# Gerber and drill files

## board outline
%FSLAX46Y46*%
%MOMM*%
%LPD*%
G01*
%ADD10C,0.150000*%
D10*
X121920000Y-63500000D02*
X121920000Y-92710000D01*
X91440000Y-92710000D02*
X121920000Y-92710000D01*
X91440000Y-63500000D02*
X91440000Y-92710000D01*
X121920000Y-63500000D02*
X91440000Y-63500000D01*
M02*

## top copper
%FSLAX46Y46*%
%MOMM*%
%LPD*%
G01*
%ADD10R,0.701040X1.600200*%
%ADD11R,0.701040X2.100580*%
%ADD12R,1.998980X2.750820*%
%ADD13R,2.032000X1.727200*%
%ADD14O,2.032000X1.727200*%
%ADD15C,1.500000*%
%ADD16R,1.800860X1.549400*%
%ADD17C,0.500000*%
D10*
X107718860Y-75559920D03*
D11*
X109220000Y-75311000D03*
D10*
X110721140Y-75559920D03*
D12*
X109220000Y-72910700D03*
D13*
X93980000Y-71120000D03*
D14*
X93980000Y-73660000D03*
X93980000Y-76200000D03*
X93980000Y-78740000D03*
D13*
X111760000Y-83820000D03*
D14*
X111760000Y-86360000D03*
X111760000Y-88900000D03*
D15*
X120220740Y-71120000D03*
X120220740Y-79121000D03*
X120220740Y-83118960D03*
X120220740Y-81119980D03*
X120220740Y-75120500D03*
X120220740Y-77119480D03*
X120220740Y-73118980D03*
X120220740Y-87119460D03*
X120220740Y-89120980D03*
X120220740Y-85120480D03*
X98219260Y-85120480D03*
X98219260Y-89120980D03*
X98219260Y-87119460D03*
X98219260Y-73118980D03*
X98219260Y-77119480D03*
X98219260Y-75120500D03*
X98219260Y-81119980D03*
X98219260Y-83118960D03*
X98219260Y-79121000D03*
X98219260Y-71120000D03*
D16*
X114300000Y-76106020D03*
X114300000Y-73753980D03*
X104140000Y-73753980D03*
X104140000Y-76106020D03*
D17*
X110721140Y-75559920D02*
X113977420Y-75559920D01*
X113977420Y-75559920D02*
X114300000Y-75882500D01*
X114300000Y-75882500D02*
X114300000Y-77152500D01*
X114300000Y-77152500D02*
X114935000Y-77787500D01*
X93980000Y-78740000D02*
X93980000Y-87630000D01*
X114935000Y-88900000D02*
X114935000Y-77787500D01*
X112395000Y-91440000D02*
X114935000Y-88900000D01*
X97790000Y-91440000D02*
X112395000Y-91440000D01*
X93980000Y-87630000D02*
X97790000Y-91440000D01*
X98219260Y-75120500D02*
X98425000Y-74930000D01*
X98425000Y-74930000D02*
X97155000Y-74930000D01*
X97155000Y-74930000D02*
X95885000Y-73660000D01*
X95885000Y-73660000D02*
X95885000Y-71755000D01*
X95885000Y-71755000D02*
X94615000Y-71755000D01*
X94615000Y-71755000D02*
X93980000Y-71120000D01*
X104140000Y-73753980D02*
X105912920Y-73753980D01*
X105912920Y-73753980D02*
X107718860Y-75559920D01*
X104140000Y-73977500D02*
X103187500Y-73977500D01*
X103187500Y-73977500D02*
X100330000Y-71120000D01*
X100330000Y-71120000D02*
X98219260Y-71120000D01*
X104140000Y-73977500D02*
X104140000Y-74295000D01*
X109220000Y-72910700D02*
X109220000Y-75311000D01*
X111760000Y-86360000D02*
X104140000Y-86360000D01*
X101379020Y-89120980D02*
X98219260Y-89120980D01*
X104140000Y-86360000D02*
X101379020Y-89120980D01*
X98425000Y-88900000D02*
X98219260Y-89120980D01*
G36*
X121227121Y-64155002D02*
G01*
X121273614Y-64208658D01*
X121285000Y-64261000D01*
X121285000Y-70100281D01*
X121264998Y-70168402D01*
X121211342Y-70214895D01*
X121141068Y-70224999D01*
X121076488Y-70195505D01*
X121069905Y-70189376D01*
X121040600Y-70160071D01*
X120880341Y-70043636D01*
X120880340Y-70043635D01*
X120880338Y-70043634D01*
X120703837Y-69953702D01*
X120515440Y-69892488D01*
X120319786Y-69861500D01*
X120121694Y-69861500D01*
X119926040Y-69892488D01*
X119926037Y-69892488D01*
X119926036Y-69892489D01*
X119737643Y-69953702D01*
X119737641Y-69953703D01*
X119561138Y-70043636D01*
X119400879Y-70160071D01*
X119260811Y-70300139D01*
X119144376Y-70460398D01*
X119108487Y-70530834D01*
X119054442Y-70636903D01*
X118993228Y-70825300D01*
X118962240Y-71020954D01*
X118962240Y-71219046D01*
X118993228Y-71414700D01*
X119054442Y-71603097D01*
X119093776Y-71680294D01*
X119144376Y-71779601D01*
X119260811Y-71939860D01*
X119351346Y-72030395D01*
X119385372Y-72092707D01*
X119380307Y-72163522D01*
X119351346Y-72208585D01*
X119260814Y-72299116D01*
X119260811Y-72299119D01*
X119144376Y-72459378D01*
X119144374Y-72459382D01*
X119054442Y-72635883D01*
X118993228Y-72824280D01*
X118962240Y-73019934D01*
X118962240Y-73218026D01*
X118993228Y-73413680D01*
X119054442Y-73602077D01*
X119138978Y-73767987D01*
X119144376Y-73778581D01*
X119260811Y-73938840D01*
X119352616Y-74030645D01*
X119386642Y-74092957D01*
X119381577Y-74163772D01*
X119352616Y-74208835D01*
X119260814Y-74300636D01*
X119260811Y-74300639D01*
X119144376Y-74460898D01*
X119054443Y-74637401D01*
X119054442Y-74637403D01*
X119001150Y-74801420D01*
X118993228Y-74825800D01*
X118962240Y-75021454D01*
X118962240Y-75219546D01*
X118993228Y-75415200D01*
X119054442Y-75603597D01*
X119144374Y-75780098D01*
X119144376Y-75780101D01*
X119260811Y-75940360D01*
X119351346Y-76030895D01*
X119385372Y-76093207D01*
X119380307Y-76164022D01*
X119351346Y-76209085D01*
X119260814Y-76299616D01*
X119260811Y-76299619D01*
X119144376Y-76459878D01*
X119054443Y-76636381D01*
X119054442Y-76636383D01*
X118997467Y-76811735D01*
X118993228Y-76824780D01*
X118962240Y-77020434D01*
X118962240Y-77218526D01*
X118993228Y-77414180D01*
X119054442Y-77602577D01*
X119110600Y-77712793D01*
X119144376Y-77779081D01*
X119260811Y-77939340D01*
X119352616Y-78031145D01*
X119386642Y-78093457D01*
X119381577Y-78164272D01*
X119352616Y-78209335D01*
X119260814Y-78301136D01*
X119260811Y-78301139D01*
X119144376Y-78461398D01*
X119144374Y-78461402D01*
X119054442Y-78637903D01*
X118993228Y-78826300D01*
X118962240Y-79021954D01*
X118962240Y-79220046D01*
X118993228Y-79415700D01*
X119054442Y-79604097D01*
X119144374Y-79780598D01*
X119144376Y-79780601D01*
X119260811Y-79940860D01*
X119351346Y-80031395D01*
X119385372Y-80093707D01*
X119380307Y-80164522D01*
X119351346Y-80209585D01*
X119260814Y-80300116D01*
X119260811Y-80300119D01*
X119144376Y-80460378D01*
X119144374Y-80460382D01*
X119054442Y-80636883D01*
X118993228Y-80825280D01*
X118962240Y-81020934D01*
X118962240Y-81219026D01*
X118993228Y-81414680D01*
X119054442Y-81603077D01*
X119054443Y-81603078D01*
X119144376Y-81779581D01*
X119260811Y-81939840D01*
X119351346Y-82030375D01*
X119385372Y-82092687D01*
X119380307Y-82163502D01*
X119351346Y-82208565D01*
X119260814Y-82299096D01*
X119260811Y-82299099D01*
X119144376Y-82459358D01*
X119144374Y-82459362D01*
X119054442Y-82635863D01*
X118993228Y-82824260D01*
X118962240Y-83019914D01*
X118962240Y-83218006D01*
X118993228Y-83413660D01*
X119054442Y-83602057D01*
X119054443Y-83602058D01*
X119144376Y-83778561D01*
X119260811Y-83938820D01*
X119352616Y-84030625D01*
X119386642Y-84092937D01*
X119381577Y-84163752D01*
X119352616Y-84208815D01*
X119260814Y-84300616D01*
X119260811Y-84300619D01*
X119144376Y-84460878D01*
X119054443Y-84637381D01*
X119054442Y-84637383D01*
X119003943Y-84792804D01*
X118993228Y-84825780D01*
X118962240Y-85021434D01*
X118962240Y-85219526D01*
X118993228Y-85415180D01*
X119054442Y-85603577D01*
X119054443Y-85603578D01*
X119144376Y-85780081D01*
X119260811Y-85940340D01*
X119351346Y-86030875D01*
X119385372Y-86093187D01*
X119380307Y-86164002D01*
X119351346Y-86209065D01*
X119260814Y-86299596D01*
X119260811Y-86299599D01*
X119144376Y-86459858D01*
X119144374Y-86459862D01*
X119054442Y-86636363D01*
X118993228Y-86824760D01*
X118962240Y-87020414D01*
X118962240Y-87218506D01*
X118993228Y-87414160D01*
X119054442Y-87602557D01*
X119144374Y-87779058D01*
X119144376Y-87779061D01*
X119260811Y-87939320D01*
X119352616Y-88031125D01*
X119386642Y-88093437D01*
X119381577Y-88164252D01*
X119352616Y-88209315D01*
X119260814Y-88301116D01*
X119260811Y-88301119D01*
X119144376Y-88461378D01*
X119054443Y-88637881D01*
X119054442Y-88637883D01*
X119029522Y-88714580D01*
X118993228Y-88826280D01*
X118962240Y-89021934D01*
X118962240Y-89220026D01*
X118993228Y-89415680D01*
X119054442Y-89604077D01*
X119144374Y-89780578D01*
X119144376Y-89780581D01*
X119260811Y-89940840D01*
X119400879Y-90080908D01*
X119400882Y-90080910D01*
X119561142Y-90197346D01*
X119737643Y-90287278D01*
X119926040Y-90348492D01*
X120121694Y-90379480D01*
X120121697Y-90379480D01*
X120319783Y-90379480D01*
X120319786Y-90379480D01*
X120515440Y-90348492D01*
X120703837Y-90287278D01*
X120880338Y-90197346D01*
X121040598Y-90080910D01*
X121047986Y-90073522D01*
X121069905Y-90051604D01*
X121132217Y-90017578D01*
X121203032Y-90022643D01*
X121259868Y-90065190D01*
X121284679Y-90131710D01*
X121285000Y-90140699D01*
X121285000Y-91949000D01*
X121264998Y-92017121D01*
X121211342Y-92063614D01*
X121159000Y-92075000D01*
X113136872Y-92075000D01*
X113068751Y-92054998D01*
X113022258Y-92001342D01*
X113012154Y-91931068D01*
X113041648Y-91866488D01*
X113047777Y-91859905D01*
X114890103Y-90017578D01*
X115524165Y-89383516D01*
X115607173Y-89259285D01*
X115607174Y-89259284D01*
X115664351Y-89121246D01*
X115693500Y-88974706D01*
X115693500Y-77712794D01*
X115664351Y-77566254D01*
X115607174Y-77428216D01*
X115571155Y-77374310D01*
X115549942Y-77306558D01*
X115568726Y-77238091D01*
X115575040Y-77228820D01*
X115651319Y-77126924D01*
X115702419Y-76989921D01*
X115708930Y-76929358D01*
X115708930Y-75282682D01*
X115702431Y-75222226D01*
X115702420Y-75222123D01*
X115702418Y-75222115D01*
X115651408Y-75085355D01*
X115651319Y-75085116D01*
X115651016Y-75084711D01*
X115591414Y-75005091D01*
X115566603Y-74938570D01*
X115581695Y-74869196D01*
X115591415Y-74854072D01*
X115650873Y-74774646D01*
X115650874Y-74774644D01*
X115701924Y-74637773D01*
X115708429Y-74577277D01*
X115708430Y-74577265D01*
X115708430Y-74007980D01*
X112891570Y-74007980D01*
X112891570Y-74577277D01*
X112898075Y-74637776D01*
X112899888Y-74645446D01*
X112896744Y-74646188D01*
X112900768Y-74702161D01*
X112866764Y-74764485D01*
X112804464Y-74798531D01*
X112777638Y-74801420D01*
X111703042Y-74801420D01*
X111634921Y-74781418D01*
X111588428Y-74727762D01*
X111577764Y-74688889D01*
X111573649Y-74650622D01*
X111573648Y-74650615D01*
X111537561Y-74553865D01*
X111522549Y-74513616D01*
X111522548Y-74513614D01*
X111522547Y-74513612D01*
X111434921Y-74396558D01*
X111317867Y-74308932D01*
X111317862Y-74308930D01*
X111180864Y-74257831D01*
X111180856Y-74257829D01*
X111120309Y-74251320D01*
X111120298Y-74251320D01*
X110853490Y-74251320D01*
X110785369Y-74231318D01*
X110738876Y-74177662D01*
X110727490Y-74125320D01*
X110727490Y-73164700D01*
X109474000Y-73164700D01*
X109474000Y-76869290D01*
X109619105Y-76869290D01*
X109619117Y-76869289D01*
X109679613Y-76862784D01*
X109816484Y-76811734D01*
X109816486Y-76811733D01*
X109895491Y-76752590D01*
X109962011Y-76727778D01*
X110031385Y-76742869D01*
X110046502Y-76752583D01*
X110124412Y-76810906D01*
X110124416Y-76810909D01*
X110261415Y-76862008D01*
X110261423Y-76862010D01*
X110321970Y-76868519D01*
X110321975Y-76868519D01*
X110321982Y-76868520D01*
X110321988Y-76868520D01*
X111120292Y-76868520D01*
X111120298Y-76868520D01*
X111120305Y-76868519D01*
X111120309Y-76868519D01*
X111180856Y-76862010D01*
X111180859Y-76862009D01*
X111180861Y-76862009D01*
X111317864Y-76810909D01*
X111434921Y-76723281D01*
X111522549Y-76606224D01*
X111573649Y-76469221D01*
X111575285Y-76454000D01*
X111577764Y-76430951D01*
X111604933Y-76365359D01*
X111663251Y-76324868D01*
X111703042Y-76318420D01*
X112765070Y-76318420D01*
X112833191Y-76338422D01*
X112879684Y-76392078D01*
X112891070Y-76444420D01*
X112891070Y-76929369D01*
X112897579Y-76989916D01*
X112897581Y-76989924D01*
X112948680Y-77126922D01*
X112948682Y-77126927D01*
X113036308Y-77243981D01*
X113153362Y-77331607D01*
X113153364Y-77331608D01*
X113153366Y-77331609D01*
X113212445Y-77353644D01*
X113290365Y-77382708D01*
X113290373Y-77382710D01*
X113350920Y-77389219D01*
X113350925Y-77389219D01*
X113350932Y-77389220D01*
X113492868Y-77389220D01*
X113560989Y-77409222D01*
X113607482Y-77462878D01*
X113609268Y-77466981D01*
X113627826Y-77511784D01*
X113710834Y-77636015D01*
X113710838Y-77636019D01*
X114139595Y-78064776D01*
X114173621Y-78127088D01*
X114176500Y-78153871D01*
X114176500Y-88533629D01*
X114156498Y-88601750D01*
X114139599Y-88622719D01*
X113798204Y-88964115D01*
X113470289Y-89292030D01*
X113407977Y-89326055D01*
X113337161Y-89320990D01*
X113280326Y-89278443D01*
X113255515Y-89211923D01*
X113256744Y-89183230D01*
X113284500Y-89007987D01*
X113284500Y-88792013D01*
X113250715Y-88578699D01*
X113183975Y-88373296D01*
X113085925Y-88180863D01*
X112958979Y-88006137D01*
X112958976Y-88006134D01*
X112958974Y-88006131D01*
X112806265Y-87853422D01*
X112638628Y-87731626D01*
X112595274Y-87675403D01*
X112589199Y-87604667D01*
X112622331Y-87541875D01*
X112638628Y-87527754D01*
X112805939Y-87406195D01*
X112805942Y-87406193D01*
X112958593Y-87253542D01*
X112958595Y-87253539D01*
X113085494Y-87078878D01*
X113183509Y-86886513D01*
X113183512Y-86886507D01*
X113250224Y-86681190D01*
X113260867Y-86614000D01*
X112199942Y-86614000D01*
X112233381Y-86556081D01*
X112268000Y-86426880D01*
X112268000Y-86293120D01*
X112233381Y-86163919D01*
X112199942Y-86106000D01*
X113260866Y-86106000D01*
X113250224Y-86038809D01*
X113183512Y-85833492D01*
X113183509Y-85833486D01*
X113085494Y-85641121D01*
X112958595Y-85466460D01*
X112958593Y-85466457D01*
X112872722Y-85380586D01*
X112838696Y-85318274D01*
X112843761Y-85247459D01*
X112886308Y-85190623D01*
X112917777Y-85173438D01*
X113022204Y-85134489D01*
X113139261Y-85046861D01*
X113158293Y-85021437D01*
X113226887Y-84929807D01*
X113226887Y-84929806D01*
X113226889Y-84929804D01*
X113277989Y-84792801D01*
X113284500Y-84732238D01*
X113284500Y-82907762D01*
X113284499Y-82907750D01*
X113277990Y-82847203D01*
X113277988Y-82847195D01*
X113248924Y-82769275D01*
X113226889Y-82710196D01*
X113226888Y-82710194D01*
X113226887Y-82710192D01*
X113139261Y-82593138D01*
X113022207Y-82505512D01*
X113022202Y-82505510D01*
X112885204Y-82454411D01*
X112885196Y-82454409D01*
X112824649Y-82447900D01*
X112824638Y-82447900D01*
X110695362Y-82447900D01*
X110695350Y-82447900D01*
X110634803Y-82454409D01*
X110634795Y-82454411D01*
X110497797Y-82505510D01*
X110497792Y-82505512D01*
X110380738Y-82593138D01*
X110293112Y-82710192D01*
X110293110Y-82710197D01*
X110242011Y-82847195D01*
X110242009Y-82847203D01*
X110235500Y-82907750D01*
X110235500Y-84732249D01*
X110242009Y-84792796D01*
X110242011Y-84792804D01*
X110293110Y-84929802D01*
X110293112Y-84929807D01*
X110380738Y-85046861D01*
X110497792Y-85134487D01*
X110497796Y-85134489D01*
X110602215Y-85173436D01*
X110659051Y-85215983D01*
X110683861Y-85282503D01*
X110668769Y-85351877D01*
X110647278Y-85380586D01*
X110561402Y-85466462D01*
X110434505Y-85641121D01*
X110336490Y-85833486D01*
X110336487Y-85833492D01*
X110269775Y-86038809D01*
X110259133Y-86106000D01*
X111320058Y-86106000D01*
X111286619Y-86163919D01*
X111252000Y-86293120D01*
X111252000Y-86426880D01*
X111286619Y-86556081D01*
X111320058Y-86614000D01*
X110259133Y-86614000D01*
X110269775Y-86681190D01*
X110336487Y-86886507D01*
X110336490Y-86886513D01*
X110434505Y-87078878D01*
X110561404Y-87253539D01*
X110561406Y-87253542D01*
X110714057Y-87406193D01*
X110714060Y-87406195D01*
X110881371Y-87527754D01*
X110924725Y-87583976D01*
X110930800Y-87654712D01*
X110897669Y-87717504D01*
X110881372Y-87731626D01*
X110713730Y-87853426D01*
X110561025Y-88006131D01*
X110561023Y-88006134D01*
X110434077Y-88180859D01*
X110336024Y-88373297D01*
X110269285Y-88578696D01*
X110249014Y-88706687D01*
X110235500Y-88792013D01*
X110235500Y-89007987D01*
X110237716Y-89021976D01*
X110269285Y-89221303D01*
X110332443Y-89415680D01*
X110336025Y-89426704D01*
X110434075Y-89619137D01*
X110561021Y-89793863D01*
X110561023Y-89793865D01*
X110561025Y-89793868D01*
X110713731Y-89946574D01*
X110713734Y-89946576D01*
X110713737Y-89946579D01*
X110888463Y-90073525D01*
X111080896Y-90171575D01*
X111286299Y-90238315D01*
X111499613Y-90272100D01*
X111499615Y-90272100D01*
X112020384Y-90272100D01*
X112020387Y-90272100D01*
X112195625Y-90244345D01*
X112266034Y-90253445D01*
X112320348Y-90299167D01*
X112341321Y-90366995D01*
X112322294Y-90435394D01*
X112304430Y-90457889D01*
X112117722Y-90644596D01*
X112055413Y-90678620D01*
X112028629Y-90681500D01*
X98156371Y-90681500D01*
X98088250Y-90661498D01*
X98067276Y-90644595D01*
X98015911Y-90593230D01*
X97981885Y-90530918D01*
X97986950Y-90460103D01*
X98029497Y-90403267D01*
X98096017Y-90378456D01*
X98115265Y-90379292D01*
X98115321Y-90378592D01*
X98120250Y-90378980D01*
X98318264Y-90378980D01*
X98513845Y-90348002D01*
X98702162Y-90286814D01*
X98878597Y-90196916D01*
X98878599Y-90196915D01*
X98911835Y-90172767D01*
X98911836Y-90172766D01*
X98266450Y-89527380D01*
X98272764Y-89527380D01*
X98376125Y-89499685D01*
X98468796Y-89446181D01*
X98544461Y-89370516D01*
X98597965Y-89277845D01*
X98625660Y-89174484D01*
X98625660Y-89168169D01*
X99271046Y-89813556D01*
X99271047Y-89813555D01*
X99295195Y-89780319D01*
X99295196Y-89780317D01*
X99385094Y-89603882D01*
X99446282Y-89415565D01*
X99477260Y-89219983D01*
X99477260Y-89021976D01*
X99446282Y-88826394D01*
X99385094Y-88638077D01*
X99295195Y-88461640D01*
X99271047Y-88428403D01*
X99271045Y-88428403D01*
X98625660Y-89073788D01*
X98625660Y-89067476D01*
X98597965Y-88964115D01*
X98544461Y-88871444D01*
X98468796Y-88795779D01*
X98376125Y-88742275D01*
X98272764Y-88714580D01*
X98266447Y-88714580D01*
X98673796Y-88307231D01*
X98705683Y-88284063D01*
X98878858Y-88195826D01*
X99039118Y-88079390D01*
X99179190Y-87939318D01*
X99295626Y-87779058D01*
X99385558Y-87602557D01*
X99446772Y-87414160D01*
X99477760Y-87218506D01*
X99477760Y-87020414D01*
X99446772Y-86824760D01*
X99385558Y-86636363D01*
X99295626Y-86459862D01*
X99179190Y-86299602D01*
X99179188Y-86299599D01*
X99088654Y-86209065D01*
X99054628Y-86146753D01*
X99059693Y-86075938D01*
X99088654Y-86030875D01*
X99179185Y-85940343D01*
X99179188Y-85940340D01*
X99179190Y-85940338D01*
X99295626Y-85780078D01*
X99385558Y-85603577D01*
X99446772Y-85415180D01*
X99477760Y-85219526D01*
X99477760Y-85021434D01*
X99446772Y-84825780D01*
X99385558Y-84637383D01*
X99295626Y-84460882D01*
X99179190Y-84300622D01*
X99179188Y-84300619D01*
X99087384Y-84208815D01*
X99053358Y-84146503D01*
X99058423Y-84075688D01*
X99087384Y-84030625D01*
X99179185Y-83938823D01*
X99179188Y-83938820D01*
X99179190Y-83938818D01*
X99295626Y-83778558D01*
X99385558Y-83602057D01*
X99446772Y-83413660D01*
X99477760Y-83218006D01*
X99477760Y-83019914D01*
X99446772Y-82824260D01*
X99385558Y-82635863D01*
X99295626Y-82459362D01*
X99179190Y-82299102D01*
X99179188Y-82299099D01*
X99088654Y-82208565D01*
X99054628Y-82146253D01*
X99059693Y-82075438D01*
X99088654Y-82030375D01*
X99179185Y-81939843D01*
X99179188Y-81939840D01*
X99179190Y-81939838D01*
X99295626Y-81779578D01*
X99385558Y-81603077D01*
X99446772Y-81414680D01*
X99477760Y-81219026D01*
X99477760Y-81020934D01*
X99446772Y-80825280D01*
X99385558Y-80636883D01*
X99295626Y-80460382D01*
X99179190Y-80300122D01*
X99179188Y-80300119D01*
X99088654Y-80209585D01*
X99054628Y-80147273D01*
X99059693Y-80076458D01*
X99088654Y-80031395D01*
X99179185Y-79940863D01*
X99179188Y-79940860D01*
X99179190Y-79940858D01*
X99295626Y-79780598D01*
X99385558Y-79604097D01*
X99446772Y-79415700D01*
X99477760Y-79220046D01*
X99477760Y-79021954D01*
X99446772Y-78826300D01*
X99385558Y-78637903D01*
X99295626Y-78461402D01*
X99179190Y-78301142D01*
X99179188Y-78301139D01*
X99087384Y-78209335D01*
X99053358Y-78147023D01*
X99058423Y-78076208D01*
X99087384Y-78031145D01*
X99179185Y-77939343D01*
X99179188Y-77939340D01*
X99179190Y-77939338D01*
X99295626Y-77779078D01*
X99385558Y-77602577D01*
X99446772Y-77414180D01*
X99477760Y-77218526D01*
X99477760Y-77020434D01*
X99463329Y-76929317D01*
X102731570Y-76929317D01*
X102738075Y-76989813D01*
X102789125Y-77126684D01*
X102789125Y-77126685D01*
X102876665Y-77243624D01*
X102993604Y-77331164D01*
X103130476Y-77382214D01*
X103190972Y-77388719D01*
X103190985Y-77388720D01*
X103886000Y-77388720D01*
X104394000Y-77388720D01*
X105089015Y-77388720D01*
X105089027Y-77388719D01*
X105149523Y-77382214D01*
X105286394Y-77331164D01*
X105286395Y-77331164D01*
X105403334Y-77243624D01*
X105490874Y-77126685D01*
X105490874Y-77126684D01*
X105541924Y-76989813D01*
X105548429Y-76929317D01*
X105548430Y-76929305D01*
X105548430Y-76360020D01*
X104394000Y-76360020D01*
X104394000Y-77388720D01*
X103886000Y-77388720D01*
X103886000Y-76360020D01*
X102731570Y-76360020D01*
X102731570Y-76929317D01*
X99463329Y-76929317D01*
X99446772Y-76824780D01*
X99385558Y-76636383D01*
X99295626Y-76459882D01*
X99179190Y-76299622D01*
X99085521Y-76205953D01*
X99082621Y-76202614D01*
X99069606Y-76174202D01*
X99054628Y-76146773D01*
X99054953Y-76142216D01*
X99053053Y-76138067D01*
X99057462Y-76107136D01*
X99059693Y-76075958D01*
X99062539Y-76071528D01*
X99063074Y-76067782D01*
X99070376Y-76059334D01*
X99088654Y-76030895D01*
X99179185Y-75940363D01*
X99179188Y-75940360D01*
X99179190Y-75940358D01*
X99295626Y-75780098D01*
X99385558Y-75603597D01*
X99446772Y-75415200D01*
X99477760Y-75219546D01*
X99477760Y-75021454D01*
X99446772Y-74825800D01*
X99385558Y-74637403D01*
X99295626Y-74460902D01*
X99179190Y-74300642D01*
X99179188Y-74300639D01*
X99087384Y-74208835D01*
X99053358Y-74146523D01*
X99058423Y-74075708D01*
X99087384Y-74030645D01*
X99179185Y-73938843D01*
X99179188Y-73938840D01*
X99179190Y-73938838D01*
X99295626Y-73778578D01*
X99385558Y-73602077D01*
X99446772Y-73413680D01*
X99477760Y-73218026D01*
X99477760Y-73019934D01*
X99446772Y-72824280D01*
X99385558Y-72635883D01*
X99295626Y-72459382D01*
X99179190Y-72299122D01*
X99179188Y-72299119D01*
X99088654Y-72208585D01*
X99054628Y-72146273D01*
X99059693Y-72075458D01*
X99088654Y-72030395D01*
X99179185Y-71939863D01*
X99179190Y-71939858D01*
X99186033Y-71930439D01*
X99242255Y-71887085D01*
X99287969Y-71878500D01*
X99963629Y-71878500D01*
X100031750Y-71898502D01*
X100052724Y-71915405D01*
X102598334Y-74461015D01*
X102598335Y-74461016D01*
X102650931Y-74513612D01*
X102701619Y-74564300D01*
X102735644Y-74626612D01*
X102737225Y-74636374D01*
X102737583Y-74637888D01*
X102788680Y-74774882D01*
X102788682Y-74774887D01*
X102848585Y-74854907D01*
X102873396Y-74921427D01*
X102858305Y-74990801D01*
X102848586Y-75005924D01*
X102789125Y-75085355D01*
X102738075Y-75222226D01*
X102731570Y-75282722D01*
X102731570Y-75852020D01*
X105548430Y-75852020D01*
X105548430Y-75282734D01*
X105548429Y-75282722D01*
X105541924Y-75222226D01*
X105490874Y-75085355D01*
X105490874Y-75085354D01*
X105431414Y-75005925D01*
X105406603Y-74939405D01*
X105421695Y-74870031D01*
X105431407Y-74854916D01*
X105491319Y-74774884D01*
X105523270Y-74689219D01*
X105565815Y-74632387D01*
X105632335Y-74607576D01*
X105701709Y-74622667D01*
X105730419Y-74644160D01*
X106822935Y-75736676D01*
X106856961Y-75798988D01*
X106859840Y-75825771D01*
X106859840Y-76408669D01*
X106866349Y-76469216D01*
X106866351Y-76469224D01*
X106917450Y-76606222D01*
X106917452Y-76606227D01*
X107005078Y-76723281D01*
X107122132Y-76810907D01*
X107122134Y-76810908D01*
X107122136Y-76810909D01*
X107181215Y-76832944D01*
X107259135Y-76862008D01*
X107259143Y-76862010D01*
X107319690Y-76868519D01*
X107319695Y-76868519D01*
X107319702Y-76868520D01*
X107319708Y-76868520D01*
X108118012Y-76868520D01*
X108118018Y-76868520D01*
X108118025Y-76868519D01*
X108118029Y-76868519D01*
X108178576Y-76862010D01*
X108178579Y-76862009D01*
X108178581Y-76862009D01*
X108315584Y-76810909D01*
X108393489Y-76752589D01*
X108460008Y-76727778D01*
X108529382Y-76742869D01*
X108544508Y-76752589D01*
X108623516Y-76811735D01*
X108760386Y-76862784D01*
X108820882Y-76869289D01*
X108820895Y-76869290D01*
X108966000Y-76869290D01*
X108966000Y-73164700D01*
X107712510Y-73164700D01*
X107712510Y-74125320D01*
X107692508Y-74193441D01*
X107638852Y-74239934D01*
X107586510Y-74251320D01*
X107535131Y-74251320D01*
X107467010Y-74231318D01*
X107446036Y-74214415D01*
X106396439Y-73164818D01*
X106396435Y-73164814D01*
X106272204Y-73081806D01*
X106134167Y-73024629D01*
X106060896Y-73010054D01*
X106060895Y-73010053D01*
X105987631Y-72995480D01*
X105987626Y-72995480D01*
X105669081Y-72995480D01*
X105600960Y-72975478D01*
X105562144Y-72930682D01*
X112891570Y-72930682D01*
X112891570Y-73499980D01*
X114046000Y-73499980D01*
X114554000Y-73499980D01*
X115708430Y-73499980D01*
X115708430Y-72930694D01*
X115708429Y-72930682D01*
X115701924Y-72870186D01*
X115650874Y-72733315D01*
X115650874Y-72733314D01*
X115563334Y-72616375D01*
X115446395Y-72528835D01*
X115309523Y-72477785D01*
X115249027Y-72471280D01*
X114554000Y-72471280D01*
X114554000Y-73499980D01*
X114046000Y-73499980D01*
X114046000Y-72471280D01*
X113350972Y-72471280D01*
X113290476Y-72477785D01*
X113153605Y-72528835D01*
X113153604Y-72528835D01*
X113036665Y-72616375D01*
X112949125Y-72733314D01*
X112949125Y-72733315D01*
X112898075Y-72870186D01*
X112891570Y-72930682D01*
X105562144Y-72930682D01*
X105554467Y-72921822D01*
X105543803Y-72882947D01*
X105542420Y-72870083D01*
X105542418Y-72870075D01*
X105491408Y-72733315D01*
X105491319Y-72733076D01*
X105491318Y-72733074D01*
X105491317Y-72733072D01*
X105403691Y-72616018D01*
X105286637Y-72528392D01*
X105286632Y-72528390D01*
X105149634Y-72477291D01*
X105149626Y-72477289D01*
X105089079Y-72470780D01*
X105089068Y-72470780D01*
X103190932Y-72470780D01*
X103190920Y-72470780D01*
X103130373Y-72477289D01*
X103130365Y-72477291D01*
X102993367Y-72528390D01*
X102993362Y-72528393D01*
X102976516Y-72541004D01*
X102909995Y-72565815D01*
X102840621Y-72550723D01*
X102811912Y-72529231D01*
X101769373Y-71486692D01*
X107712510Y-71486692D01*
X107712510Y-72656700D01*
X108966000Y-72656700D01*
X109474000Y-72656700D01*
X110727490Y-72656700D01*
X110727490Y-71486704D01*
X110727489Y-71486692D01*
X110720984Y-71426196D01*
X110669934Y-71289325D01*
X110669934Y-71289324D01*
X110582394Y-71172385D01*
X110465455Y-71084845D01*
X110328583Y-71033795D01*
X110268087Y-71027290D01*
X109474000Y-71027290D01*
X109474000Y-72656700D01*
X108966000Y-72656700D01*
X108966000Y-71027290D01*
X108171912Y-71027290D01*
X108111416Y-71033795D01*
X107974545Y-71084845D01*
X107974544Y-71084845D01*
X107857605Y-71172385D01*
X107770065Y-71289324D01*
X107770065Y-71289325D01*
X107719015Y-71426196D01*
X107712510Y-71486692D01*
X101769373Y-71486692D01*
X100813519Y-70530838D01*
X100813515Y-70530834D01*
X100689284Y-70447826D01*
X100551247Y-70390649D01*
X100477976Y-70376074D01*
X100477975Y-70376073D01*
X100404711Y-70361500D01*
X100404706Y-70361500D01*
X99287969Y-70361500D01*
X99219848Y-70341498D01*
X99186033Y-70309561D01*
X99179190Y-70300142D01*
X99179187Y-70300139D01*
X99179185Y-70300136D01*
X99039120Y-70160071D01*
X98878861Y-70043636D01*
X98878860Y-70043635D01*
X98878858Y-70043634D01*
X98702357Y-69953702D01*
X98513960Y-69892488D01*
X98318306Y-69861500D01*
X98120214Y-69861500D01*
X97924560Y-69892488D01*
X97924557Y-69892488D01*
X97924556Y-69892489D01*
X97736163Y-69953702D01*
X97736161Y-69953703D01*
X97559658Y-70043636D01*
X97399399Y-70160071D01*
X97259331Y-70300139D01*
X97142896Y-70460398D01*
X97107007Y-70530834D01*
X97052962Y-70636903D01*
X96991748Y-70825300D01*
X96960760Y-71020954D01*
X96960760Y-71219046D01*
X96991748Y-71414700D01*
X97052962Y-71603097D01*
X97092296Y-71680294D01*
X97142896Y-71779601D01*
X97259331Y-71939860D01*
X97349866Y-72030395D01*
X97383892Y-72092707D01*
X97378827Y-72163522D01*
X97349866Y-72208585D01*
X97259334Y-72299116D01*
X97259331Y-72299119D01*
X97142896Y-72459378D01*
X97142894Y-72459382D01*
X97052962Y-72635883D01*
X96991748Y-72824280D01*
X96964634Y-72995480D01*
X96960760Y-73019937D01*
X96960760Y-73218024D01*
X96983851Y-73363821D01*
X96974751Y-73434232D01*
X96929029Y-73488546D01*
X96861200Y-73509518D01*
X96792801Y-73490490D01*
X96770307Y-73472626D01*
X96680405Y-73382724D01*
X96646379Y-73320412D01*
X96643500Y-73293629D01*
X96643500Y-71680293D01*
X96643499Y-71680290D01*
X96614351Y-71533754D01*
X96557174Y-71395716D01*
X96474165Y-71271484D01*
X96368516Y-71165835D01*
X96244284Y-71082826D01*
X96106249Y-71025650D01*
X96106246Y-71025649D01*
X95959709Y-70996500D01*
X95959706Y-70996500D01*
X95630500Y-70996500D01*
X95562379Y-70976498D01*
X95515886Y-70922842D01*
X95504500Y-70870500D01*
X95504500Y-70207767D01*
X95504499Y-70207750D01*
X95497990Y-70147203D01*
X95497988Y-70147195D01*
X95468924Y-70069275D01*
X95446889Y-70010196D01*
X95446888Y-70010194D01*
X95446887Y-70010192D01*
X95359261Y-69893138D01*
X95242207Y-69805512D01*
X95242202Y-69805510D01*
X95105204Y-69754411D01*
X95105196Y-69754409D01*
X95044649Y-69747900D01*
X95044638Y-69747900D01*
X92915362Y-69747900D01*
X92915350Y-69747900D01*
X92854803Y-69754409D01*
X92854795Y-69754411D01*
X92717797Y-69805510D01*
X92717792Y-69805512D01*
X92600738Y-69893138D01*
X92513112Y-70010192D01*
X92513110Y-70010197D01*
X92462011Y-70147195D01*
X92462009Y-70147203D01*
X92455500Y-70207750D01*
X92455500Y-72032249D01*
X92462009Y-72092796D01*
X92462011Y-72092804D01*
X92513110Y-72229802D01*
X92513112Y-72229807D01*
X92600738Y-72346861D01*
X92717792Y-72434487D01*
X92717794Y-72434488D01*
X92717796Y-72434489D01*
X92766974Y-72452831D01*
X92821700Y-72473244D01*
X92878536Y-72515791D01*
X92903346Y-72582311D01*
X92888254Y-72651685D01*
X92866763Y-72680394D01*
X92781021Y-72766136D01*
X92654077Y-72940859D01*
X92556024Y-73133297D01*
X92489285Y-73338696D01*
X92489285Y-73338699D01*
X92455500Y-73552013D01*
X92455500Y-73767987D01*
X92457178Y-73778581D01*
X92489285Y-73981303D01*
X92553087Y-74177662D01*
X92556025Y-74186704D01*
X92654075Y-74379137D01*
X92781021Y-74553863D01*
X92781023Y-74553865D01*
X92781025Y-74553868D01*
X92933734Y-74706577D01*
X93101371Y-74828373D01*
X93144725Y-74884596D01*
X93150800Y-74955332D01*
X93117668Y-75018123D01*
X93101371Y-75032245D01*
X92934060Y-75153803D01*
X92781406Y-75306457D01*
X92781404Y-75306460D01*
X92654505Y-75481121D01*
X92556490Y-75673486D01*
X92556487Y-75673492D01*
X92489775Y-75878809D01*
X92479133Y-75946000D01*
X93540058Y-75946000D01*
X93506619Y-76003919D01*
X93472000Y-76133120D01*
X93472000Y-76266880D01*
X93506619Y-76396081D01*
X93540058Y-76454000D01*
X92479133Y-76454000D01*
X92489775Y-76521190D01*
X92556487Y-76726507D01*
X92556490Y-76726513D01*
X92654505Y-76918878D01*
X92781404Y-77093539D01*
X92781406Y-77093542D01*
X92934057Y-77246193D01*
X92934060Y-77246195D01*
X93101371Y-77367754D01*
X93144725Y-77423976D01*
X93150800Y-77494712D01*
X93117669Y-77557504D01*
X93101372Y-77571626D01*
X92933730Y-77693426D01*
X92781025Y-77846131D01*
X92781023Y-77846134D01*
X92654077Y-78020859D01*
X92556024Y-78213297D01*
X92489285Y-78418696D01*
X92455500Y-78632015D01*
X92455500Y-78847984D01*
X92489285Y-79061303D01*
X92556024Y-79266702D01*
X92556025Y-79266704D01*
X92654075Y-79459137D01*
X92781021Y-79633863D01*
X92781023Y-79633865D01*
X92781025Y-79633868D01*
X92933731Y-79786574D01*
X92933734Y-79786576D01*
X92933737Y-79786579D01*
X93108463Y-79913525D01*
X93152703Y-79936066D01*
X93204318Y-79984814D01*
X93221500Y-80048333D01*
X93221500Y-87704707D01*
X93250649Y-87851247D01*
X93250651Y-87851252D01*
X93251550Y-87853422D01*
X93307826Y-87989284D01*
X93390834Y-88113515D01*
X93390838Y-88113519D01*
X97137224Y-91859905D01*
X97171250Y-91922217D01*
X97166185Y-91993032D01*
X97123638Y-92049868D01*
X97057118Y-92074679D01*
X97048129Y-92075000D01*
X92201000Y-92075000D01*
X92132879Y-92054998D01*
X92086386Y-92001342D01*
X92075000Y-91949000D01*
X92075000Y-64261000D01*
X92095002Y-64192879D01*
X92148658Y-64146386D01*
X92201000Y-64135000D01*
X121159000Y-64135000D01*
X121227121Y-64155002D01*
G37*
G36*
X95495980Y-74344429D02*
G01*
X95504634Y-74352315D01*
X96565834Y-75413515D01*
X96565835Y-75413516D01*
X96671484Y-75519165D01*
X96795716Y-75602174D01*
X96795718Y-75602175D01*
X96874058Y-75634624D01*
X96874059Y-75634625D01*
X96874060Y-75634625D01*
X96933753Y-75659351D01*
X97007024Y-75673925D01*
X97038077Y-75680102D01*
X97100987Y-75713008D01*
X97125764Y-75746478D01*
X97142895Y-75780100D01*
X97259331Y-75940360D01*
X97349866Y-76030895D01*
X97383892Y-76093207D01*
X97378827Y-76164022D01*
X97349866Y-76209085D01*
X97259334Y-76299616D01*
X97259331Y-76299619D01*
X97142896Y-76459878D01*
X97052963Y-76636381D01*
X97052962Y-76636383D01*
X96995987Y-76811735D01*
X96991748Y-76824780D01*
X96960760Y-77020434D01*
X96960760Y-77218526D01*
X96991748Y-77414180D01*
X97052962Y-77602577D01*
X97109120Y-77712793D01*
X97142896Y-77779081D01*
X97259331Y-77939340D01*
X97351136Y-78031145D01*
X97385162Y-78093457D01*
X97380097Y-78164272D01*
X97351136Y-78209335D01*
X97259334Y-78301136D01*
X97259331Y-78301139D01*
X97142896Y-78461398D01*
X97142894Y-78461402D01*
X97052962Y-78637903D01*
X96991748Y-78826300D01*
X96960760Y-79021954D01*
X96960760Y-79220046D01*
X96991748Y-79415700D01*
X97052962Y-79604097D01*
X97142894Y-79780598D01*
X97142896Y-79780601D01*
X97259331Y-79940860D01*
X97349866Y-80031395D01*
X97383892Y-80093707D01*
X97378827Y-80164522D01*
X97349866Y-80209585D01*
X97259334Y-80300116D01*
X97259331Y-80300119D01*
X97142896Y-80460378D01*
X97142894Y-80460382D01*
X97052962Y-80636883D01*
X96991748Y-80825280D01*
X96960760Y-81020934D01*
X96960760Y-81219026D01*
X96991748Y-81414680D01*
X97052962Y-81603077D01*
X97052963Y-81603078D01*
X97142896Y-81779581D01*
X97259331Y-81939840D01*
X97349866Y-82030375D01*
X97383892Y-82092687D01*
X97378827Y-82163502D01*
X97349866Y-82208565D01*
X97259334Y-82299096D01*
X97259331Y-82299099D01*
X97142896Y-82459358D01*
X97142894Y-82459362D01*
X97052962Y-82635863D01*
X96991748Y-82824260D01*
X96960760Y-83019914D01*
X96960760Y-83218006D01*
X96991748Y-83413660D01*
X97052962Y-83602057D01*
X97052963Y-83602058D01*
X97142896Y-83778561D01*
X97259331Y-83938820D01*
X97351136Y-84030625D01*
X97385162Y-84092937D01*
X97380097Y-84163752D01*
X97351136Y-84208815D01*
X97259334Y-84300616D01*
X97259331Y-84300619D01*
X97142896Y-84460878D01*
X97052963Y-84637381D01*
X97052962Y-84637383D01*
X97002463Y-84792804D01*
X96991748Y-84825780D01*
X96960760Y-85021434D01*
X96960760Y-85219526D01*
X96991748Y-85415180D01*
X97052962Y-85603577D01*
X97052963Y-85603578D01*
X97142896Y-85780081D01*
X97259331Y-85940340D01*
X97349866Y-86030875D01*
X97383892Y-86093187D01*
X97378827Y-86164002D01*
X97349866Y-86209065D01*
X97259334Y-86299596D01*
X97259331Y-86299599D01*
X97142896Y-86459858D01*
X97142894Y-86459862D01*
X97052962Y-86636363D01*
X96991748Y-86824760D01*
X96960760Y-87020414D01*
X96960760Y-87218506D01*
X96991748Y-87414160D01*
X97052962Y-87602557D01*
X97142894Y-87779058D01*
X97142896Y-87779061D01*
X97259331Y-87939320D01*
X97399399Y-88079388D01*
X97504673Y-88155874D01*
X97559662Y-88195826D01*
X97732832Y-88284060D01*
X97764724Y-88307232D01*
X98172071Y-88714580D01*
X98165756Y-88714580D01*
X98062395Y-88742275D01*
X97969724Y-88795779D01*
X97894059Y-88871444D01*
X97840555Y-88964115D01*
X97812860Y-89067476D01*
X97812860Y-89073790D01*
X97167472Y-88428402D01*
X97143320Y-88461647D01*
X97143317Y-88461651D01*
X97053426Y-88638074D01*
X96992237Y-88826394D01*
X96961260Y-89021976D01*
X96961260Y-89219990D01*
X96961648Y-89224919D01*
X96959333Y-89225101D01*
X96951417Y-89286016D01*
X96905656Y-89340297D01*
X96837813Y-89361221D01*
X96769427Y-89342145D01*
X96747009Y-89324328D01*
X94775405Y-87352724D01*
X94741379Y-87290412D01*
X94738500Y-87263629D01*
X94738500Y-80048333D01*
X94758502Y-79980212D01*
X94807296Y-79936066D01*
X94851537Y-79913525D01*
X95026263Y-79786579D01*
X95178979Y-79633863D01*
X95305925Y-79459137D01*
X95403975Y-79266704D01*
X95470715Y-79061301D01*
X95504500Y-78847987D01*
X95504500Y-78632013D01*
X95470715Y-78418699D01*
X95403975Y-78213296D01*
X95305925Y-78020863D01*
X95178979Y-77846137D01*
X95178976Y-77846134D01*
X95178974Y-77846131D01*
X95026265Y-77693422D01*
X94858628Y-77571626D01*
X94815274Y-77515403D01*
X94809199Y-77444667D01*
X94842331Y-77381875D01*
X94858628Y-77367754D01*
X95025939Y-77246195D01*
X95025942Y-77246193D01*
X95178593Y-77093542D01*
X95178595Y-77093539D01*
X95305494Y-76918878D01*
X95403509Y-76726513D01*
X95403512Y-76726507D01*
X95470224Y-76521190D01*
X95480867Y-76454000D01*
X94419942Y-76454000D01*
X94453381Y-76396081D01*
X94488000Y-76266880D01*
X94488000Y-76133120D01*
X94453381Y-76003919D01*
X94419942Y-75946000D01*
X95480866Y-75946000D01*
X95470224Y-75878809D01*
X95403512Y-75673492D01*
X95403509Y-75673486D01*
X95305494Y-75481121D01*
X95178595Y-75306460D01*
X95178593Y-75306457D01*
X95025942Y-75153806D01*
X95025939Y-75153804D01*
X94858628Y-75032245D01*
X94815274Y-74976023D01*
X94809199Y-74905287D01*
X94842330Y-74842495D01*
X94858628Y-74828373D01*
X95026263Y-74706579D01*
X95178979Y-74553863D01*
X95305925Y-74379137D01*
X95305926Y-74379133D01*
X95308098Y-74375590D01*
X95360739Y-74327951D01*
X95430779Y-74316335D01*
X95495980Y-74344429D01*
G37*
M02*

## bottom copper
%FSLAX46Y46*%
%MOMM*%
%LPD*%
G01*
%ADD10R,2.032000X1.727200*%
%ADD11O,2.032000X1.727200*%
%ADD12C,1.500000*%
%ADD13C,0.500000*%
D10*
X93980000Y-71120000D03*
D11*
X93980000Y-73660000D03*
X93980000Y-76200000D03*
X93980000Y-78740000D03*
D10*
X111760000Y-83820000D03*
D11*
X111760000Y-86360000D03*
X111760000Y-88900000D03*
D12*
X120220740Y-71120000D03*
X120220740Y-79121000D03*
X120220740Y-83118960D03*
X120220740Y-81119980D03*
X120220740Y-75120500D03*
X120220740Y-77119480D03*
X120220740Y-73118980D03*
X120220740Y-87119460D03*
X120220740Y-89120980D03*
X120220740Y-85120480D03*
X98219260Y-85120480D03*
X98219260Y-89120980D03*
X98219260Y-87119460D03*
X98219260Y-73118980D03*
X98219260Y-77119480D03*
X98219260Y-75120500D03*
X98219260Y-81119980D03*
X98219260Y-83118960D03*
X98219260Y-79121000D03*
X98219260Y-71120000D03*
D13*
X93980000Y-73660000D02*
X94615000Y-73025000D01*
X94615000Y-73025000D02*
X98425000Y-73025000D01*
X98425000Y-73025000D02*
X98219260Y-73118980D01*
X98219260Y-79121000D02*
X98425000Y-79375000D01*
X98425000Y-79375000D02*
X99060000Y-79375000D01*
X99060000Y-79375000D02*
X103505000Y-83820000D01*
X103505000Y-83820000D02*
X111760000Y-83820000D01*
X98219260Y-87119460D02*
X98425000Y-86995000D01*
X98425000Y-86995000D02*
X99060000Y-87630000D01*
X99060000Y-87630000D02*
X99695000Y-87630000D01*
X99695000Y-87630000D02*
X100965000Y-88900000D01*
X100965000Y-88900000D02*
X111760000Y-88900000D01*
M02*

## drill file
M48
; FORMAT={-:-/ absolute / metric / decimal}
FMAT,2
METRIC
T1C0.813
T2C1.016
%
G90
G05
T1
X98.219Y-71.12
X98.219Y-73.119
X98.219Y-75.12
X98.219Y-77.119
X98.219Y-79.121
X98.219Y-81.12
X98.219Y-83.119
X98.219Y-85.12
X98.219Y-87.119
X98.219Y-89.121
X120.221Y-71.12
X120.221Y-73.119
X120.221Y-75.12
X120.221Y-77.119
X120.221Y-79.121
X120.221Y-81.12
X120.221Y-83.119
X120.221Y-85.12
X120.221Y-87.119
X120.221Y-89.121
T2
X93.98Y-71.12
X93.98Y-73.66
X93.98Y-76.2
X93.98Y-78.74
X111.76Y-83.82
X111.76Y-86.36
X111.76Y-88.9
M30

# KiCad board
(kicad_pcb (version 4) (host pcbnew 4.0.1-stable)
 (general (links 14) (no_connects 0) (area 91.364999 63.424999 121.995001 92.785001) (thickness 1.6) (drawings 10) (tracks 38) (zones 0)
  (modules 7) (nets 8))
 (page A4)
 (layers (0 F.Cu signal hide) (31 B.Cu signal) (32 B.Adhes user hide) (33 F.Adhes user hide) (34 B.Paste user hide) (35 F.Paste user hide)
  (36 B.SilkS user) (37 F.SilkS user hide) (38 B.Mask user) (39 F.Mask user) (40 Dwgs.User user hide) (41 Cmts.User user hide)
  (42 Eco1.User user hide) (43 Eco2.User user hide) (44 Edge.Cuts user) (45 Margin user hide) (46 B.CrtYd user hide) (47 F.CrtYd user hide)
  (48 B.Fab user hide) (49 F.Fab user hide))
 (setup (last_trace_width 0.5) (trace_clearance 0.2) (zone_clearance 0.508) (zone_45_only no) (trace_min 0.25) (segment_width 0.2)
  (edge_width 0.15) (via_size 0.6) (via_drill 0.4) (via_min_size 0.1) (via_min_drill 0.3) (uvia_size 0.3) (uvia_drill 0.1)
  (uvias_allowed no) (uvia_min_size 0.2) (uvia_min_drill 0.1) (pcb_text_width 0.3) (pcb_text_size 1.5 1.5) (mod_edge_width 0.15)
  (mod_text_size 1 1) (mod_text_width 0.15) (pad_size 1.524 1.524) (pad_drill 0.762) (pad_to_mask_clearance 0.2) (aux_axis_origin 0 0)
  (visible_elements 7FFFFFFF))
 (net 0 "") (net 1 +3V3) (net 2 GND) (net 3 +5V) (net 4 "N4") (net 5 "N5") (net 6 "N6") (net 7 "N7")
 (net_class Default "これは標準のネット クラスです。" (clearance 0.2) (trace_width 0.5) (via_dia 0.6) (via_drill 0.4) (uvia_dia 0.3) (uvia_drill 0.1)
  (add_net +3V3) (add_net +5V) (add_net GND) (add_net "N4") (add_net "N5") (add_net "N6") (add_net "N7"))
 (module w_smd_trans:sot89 (layer F.Cu) (at 109.22 73.66)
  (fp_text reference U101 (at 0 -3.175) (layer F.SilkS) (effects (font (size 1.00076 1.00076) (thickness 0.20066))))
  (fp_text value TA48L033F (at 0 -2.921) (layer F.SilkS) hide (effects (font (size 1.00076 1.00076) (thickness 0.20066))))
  (pad 1 smd rect (at -1.50114 1.89992) (size 0.70104 1.6002) (layers F.Cu F.Paste F.Mask) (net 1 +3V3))
  (pad 2 smd rect (at 0 1.651) (size 0.70104 2.10058) (layers F.Cu F.Paste F.Mask) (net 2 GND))
  (pad 3 smd rect (at 1.50114 1.89992) (size 0.70104 1.6002) (layers F.Cu F.Paste F.Mask) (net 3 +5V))
  (pad 2 smd rect (at 0 -0.7493) (size 1.99898 2.75082) (layers F.Cu F.Paste F.Mask) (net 2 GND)))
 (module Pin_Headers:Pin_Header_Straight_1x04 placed (layer B.Cu) (at 93.98 71.12 180)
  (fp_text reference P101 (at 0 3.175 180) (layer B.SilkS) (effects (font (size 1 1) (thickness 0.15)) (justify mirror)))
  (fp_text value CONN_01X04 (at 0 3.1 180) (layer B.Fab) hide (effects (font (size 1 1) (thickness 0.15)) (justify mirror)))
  (pad 1 thru_hole rect (at 0 0 180) (size 2.032 1.7272) (drill 1.016) (layers *.Cu *.Mask B.SilkS) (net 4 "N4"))
  (pad 2 thru_hole oval (at 0 -2.54 180) (size 2.032 1.7272) (drill 1.016) (layers *.Cu *.Mask B.SilkS) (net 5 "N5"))
  (pad 3 thru_hole oval (at 0 -5.08 180) (size 2.032 1.7272) (drill 1.016) (layers *.Cu *.Mask B.SilkS) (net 2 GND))
  (pad 4 thru_hole oval (at 0 -7.62 180) (size 2.032 1.7272) (drill 1.016) (layers *.Cu *.Mask B.SilkS) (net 3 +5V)))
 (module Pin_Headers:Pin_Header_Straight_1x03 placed (layer B.Cu) (at 111.76 83.82 180)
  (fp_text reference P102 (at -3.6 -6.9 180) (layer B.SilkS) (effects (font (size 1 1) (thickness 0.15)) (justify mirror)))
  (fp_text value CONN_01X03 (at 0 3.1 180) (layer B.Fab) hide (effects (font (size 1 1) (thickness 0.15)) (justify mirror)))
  (pad 1 thru_hole rect (at 0 0 180) (size 2.032 1.7272) (drill 1.016) (layers *.Cu *.Mask B.SilkS) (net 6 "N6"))
  (pad 2 thru_hole oval (at 0 -2.54 180) (size 2.032 1.7272) (drill 1.016) (layers *.Cu *.Mask B.SilkS) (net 2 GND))
  (pad 3 thru_hole oval (at 0 -5.08 180) (size 2.032 1.7272) (drill 1.016) (layers *.Cu *.Mask B.SilkS) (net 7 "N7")))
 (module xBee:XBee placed (layer F.Cu) (at 109.22 71.12)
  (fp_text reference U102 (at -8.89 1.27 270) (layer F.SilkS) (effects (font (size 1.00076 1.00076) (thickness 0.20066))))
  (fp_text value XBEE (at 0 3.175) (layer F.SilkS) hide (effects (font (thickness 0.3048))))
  (pad 20 thru_hole circle (at 11.00074 0) (size 1.5 1.5) (drill 0.8128) (layers *.Cu))
  (pad 16 thru_hole circle (at 11.00074 8.001) (size 1.5 1.5) (drill 0.8128) (layers *.Cu))
  (pad 14 thru_hole circle (at 11.00074 11.99896) (size 1.5 1.5) (drill 0.8128) (layers *.Cu))
  (pad 15 thru_hole circle (at 11.00074 9.99998) (size 1.5 1.5) (drill 0.8128) (layers *.Cu))
  (pad 18 thru_hole circle (at 11.00074 4.0005) (size 1.5 1.5) (drill 0.8128) (layers *.Cu))
  (pad 17 thru_hole circle (at 11.00074 5.99948) (size 1.5 1.5) (drill 0.8128) (layers *.Cu))
  (pad 19 thru_hole circle (at 11.00074 1.99898) (size 1.5 1.5) (drill 0.8128) (layers *.Cu))
  (pad 12 thru_hole circle (at 11.00074 15.99946) (size 1.5 1.5) (drill 0.8128) (layers *.Cu))
  (pad 11 thru_hole circle (at 11.00074 18.00098) (size 1.5 1.5) (drill 0.8128) (layers *.Cu))
  (pad 13 thru_hole circle (at 11.00074 14.00048) (size 1.5 1.5) (drill 0.8128) (layers *.Cu))
  (pad 8 thru_hole circle (at -11.00074 14.00048) (size 1.5 1.5) (drill 0.8128) (layers *.Cu))
  (pad 10 thru_hole circle (at -11.00074 18.00098) (size 1.5 1.5) (drill 0.8128) (layers *.Cu) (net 2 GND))
  (pad 9 thru_hole circle (at -11.00074 15.99946) (size 1.5 1.5) (drill 0.8128) (layers *.Cu) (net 7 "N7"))
  (pad 2 thru_hole circle (at -11.00074 1.99898) (size 1.5 1.5) (drill 0.8128) (layers *.Cu) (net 5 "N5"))
  (pad 4 thru_hole circle (at -11.00074 5.99948) (size 1.5 1.5) (drill 0.8128) (layers *.Cu))
  (pad 3 thru_hole circle (at -11.00074 4.0005) (size 1.5 1.5) (drill 0.8128) (layers *.Cu) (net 4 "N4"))
  (pad 6 thru_hole circle (at -11.00074 9.99998) (size 1.5 1.5) (drill 0.8128) (layers *.Cu))
  (pad 7 thru_hole circle (at -11.00074 11.99896) (size 1.5 1.5) (drill 0.8128) (layers *.Cu))
  (pad 5 thru_hole circle (at -11.00074 8.001) (size 1.5 1.5) (drill 0.8128) (layers *.Cu) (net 6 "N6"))
  (pad 1 thru_hole circle (at -11.00074 0) (size 1.5 1.5) (drill 0.8128) (layers *.Cu) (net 1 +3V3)))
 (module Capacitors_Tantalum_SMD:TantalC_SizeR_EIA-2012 (layer F.Cu) (at 114.3 74.93 270)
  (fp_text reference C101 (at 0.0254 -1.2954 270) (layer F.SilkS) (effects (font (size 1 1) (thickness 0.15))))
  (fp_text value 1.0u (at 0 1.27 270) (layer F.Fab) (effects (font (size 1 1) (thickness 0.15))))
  (pad 1 smd rect (at 1.17602 0 270) (size 1.5494 1.80086) (layers F.Cu F.Paste F.Mask) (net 3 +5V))
  (pad 2 smd rect (at -1.17602 0 270) (size 1.5494 1.80086) (layers F.Cu F.Paste F.Mask) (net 2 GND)))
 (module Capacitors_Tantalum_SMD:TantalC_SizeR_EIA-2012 (layer F.Cu) (at 104.14 74.93 90)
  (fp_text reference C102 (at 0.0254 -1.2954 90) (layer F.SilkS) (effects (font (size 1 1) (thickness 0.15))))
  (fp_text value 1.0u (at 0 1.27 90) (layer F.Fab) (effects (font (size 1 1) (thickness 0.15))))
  (pad 1 smd rect (at 1.17602 0 90) (size 1.5494 1.80086) (layers F.Cu F.Paste F.Mask) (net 1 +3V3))
  (pad 2 smd rect (at -1.17602 0 90) (size 1.5494 1.80086) (layers F.Cu F.Paste F.Mask) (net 2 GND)))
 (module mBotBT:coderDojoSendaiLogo (layer B.Cu) (at 107.442 73.152 180)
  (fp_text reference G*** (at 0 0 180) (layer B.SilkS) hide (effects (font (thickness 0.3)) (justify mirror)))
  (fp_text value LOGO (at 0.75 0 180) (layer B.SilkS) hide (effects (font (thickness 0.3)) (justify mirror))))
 (gr_line (start 121.92 63.5) (end 121.92 92.71) (angle 90) (layer Edge.Cuts) (width 0.15))
 (gr_line (start 91.44 92.71) (end 121.92 92.71) (angle 90) (layer Edge.Cuts) (width 0.15))
 (gr_line (start 91.44 63.5) (end 91.44 92.71) (angle 90) (layer Edge.Cuts) (width 0.15))
 (gr_line (start 121.92 63.5) (end 91.44 63.5) (angle 90) (layer Edge.Cuts) (width 0.15))
 (segment (start 110.72114 75.55992) (end 113.97742 75.55992) (width 0.5) (layer F.Cu) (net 3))
 (segment (start 113.97742 75.55992) (end 114.3 75.8825) (width 0.5) (layer F.Cu) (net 3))
 (segment (start 114.3 75.8825) (end 114.3 77.1525) (width 0.5) (layer F.Cu) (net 3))
 (segment (start 114.3 77.1525) (end 114.935 77.7875) (width 0.5) (layer F.Cu) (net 3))
 (segment (start 93.98 78.74) (end 93.98 87.63) (width 0.5) (layer F.Cu) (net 3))
 (segment (start 114.935 88.9) (end 114.935 77.7875) (width 0.5) (layer F.Cu) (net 3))
 (segment (start 112.395 91.44) (end 114.935 88.9) (width 0.5) (layer F.Cu) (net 3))
 (segment (start 97.79 91.44) (end 112.395 91.44) (width 0.5) (layer F.Cu) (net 3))
 (segment (start 93.98 87.63) (end 97.79 91.44) (width 0.5) (layer F.Cu) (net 3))
 (segment (start 98.21926 75.1205) (end 98.425 74.93) (width 0.5) (layer F.Cu) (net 4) (status 80000))
 (segment (start 98.425 74.93) (end 97.155 74.93) (width 0.5) (layer F.Cu) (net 4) (status 80000))
 (segment (start 97.155 74.93) (end 95.885 73.66) (width 0.5) (layer F.Cu) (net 4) (status 80000))
 (segment (start 95.885 73.66) (end 95.885 71.755) (width 0.5) (layer F.Cu) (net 4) (status 80000))
 (segment (start 95.885 71.755) (end 94.615 71.755) (width 0.5) (layer F.Cu) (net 4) (status 80000))
 (segment (start 94.615 71.755) (end 93.98 71.12) (width 0.5) (layer F.Cu) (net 4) (status 80000))
 (segment (start 93.98 73.66) (end 94.615 73.025) (width 0.5) (layer B.Cu) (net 5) (status 80000))
 (segment (start 94.615 73.025) (end 98.425 73.025) (width 0.5) (layer B.Cu) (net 5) (status 80000))
 (segment (start 98.425 73.025) (end 98.21926 73.11898) (width 0.5) (layer B.Cu) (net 5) (status 80000))
 (segment (start 98.21926 79.121) (end 98.425 79.375) (width 0.5) (layer B.Cu) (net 6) (status 80000))
 (segment (start 98.425 79.375) (end 99.06 79.375) (width 0.5) (layer B.Cu) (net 6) (status 80000))
 (segment (start 99.06 79.375) (end 103.505 83.82) (width 0.5) (layer B.Cu) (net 6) (status 80000))
 (segment (start 103.505 83.82) (end 111.76 83.82) (width 0.5) (layer B.Cu) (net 6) (status 80000))
 (segment (start 98.21926 87.11946) (end 98.425 86.995) (width 0.5) (layer B.Cu) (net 7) (status 80000))
 (segment (start 98.425 86.995) (end 99.06 87.63) (width 0.5) (layer B.Cu) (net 7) (status 80000))
 (segment (start 99.06 87.63) (end 99.695 87.63) (width 0.5) (layer B.Cu) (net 7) (status 80000))
 (segment (start 99.695 87.63) (end 100.965 88.9) (width 0.5) (layer B.Cu) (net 7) (status 80000))
 (segment (start 100.965 88.9) (end 111.76 88.9) (width 0.5) (layer B.Cu) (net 7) (status 80000))
 (segment (start 104.14 73.75398) (end 105.91292 73.75398) (width 0.5) (layer F.Cu) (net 1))
 (segment (start 105.91292 73.75398) (end 107.71886 75.55992) (width 0.5) (layer F.Cu) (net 1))
 (segment (start 104.14 73.9775) (end 103.1875 73.9775) (width 0.5) (layer F.Cu) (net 1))
 (segment (start 103.1875 73.9775) (end 100.33 71.12) (width 0.5) (layer F.Cu) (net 1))
 (segment (start 100.33 71.12) (end 98.21926 71.12) (width 0.5) (layer F.Cu) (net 1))
 (segment (start 104.14 73.9775) (end 104.14 74.295) (width 0.5) (layer F.Cu) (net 1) (status 80000))
 (segment (start 109.22 72.9107) (end 109.22 75.311) (width 0.5) (layer F.Cu) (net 2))
 (segment (start 111.76 86.36) (end 104.14 86.36) (width 0.5) (layer F.Cu) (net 2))
 (segment (start 101.37902 89.12098) (end 98.21926 89.12098) (width 0.5) (layer F.Cu) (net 2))
 (segment (start 104.14 86.36) (end 101.37902 89.12098) (width 0.5) (layer F.Cu) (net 2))
 (segment (start 98.425 88.9) (end 98.21926 89.12098) (width 0.5) (layer F.Cu) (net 2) (status 80000))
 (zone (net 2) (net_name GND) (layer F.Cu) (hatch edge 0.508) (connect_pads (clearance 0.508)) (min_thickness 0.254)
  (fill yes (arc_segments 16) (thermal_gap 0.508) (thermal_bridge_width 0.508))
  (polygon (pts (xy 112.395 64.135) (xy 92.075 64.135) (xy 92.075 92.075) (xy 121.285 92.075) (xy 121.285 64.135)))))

